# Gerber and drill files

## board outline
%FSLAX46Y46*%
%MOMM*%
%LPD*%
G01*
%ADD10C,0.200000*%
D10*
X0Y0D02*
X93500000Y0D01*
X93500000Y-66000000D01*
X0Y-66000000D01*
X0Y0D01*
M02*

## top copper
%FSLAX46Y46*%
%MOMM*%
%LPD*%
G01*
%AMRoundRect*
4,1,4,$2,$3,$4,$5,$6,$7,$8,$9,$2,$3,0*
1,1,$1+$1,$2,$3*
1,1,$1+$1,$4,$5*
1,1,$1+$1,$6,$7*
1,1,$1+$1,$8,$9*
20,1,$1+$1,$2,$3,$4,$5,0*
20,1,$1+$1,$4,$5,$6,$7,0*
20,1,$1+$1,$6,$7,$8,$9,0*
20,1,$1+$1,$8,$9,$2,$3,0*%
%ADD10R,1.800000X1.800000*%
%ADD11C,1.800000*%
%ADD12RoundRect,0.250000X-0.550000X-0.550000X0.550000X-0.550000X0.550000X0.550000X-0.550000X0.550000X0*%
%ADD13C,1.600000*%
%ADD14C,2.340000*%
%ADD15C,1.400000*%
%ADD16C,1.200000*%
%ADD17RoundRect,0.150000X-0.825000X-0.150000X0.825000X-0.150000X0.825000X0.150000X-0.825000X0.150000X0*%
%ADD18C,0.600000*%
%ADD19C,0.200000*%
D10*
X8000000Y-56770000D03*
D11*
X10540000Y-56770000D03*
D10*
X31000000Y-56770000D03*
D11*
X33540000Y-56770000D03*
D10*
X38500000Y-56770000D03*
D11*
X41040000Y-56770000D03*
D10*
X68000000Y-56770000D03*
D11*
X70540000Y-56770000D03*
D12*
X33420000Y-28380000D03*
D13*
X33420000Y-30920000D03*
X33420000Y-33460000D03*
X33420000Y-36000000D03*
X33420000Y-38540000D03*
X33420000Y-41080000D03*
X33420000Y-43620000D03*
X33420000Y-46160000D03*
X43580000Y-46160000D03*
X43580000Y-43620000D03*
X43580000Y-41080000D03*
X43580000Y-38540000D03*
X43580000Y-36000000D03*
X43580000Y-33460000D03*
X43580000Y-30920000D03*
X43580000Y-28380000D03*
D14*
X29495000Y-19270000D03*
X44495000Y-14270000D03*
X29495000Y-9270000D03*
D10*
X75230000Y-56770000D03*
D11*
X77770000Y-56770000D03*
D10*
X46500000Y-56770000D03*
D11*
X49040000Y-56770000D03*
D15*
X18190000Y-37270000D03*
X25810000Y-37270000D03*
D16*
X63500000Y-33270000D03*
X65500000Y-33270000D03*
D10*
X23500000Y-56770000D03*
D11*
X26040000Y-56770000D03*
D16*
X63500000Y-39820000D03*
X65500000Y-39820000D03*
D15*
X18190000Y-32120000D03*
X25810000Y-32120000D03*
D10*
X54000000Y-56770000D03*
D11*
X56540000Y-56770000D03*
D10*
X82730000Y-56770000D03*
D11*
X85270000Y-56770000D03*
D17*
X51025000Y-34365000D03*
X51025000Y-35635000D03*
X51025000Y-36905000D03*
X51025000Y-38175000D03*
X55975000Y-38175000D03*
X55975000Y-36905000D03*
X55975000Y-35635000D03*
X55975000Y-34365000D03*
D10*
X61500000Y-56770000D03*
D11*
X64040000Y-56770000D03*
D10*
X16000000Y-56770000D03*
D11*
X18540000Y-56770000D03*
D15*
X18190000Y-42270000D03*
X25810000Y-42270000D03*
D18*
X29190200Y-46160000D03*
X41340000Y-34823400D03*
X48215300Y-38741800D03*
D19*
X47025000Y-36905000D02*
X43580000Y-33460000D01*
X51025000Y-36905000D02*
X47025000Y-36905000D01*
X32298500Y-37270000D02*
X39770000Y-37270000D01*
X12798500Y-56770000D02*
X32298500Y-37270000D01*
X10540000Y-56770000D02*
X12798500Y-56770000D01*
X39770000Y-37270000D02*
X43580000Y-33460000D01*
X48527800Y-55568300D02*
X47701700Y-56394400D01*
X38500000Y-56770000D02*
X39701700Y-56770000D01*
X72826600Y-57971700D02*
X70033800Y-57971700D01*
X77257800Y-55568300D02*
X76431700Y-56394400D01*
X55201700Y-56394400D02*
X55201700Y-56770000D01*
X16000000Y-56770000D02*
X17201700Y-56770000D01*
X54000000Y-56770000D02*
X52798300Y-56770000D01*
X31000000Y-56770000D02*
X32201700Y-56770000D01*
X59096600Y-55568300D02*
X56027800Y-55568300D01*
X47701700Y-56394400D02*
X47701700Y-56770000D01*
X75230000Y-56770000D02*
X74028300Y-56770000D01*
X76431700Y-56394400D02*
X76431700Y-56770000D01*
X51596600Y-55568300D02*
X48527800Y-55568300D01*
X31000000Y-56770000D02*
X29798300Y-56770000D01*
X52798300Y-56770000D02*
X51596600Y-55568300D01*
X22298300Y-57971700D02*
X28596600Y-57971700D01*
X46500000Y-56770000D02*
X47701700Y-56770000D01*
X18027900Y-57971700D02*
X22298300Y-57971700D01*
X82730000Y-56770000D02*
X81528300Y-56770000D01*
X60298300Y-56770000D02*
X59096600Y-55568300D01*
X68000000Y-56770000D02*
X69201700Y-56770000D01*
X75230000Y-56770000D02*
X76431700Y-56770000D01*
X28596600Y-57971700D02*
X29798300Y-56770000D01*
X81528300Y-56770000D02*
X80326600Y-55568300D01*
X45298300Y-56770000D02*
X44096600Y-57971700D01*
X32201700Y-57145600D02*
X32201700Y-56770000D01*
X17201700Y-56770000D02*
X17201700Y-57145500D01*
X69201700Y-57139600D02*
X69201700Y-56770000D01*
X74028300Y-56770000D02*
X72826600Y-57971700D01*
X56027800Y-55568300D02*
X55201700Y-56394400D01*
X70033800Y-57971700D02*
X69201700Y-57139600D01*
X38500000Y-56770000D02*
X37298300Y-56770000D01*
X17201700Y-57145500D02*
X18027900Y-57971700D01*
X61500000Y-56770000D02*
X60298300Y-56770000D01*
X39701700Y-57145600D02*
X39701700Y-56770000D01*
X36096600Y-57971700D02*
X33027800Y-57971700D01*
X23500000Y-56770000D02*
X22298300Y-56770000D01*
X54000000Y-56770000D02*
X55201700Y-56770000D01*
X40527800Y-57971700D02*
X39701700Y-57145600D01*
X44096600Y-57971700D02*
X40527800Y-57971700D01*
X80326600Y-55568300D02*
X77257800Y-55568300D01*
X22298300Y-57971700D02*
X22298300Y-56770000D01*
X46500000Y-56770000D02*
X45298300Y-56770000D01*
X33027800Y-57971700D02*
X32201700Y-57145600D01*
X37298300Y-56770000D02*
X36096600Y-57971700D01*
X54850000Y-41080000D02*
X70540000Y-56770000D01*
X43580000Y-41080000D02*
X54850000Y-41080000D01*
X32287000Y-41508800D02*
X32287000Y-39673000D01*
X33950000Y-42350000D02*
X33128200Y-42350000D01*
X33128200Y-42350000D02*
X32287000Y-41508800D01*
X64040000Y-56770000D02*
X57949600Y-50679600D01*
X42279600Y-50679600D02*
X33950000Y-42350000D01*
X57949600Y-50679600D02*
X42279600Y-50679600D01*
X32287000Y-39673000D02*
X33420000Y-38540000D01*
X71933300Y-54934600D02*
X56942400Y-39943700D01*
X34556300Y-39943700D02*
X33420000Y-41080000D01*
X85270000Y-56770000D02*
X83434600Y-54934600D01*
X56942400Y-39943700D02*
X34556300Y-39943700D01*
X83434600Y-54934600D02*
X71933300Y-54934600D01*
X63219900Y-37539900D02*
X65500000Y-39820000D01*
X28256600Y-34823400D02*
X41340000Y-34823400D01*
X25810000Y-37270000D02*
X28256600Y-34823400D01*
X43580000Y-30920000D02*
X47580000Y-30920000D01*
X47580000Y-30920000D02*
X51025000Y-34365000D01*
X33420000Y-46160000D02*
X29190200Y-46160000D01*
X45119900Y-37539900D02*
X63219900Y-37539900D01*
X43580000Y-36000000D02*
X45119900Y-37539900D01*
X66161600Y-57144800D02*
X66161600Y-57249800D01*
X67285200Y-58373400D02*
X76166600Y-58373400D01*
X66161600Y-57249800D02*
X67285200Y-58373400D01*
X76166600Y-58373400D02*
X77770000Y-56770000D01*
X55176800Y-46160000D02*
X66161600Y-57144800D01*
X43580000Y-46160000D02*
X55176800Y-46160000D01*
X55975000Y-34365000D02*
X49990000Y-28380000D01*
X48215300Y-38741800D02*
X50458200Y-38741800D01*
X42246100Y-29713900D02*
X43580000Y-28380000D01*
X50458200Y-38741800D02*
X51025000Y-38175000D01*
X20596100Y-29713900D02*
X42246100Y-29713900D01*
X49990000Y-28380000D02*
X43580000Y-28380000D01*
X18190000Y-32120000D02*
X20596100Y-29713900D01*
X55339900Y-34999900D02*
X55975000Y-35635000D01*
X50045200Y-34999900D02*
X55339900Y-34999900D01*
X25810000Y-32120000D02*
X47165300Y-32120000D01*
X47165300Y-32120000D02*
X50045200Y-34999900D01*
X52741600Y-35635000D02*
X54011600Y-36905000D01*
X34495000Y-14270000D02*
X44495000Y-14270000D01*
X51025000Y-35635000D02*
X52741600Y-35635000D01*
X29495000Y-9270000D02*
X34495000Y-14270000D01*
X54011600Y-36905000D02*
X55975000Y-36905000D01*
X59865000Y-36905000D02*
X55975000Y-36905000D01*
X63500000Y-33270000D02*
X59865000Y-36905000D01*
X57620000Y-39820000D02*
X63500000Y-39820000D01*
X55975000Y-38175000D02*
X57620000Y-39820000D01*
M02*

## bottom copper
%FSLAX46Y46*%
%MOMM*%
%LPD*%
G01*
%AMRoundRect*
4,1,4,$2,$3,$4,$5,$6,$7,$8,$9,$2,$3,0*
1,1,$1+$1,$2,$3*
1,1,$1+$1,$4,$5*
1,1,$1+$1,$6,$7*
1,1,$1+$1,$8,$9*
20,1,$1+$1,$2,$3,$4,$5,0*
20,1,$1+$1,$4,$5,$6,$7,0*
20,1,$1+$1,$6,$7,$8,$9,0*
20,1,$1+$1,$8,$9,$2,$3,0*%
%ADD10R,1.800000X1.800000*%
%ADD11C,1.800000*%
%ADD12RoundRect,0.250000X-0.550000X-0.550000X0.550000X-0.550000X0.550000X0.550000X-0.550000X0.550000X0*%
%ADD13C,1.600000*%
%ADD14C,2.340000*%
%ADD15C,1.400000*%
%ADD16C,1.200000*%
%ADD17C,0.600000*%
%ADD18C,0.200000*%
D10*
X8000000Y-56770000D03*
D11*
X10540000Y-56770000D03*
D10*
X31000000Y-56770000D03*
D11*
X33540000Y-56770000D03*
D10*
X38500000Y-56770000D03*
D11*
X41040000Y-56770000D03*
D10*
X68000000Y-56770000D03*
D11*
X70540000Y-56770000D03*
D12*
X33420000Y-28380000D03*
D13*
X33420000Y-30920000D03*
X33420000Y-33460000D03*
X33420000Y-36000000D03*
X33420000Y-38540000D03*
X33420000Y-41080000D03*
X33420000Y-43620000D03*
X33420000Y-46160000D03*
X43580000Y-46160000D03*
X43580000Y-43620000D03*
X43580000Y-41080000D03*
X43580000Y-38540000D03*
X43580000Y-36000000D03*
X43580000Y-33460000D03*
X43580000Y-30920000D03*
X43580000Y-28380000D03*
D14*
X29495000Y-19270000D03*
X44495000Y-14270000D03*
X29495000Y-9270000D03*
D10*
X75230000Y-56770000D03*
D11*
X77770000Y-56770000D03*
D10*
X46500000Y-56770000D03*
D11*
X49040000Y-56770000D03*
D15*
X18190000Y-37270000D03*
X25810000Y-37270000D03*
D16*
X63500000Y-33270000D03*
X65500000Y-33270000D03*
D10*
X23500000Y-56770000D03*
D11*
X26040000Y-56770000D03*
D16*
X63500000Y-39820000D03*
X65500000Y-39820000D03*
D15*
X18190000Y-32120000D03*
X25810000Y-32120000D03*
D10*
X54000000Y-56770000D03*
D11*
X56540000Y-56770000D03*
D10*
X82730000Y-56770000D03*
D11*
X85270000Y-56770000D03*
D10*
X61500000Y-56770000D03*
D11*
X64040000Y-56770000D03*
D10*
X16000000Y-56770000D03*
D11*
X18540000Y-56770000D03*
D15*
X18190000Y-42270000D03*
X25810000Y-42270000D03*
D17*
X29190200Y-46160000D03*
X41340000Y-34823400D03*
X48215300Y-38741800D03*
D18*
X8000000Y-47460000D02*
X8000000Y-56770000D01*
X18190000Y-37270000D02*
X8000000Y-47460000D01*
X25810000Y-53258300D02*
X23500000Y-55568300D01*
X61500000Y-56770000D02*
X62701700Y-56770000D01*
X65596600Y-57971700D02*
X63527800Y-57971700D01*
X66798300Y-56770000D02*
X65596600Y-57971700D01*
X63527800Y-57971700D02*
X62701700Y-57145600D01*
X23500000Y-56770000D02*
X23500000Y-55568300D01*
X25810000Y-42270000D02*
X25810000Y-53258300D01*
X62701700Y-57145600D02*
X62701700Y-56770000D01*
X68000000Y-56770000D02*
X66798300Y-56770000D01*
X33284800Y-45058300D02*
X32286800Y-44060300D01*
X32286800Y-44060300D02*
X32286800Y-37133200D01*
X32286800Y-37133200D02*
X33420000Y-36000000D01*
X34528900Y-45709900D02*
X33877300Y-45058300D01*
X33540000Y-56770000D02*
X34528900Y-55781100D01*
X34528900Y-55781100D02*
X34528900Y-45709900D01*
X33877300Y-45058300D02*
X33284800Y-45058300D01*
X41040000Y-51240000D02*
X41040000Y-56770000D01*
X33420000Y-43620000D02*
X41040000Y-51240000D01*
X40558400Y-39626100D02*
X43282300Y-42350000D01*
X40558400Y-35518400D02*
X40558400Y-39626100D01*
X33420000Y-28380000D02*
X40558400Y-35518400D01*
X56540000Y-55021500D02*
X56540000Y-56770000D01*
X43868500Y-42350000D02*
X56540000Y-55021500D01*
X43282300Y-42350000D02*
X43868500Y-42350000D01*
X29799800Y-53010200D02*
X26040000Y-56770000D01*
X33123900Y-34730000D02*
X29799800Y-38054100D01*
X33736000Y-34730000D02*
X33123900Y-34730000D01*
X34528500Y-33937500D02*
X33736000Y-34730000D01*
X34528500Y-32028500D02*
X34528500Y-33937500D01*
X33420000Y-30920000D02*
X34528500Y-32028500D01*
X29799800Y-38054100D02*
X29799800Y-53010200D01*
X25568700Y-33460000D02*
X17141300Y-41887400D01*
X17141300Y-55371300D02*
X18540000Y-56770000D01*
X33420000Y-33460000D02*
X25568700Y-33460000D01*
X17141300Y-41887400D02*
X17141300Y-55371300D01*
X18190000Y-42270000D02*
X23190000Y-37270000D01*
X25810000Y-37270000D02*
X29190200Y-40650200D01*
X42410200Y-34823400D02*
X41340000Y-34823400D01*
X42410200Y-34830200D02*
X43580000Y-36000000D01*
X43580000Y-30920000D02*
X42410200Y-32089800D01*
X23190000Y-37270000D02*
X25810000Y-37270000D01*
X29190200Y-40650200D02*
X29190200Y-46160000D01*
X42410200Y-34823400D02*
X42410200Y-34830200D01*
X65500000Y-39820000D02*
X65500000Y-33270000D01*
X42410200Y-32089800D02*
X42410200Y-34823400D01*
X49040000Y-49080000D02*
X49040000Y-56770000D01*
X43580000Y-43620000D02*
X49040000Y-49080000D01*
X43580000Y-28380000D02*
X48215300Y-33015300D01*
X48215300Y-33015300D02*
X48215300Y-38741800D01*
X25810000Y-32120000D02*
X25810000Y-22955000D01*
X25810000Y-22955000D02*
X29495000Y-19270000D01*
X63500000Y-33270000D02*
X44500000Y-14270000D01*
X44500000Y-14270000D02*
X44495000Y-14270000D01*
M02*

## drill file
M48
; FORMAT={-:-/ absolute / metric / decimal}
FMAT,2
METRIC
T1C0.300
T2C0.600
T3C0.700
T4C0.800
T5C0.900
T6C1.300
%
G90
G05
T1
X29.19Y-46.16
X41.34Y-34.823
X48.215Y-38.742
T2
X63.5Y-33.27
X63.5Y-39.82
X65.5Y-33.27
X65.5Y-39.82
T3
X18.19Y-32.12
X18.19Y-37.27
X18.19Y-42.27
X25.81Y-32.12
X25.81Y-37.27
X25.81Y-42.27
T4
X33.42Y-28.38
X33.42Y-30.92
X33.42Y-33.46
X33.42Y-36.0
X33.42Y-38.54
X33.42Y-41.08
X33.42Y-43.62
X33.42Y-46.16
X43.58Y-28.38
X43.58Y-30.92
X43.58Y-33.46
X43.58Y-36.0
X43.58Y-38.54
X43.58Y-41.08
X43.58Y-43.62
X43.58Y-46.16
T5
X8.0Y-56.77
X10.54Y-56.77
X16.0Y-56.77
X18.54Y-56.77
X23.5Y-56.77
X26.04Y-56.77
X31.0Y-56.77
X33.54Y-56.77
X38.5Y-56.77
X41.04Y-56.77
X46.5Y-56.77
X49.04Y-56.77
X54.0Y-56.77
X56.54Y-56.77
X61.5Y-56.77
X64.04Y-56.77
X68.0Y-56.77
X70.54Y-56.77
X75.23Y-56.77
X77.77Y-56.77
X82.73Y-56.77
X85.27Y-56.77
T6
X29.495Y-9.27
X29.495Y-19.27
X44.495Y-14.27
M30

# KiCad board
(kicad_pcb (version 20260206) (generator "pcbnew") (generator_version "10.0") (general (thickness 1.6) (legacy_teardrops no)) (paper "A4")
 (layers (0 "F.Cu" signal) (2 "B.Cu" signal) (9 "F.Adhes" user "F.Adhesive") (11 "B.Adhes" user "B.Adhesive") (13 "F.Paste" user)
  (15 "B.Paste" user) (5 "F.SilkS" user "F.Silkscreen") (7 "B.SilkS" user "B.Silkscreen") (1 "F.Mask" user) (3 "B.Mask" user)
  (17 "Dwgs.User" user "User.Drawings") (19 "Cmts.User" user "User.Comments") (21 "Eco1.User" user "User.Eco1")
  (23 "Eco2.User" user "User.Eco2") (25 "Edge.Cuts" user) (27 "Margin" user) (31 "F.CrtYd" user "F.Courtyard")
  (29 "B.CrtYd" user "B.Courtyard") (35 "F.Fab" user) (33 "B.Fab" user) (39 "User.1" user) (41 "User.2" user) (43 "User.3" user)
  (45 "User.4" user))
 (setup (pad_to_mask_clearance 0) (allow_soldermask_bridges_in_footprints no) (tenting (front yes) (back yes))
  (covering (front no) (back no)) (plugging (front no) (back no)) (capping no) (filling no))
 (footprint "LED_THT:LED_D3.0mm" (layer "F.Cu") (at 8 56.77)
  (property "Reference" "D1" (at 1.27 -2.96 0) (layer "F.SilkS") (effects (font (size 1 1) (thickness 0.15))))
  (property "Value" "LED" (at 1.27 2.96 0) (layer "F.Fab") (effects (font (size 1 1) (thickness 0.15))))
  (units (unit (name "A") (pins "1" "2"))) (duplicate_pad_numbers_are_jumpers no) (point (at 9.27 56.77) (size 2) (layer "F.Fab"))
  (pad "1" thru_hole rect (at 0 0) (size 1.8 1.8) (drill 0.9) (layers "*.Cu" "*.Mask") (remove_unused_layers no) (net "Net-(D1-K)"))
  (pad "2" thru_hole circle (at 2.54 0) (size 1.8 1.8) (drill 0.9) (layers "*.Cu" "*.Mask") (remove_unused_layers no) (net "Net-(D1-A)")))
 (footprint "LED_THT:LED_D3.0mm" (layer "F.Cu") (at 31 56.77)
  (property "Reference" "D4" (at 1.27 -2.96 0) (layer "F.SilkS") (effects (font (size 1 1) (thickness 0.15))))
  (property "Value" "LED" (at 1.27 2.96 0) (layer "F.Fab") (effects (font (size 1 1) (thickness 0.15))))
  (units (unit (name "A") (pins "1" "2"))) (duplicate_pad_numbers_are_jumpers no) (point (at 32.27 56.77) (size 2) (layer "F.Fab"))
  (pad "1" thru_hole rect (at 0 0) (size 1.8 1.8) (drill 0.9) (layers "*.Cu" "*.Mask") (remove_unused_layers no) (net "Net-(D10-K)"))
  (pad "2" thru_hole circle (at 2.54 0) (size 1.8 1.8) (drill 0.9) (layers "*.Cu" "*.Mask") (remove_unused_layers no) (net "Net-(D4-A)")))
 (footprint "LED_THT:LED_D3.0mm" (layer "F.Cu") (at 38.5 56.77)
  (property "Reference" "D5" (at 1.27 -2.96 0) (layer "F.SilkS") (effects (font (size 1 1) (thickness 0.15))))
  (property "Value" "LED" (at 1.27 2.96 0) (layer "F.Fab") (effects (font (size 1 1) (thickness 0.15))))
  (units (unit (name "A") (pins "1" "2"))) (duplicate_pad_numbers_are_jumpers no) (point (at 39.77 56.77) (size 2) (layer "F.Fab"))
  (pad "1" thru_hole rect (at 0 0) (size 1.8 1.8) (drill 0.9) (layers "*.Cu" "*.Mask") (remove_unused_layers no) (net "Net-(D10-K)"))
  (pad "2" thru_hole circle (at 2.54 0) (size 1.8 1.8) (drill 0.9) (layers "*.Cu" "*.Mask") (remove_unused_layers no) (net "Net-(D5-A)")))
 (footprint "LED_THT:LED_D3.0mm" (layer "F.Cu") (at 68 56.77)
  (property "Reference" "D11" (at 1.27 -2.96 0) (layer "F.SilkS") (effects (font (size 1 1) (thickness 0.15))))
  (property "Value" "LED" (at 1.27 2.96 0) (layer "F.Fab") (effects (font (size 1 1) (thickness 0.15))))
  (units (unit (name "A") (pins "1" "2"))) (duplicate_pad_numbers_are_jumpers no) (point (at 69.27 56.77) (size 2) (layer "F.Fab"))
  (pad "1" thru_hole rect (at 0 0) (size 1.8 1.8) (drill 0.9) (layers "*.Cu" "*.Mask") (remove_unused_layers no) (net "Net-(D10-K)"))
  (pad "2" thru_hole circle (at 2.54 0) (size 1.8 1.8) (drill 0.9) (layers "*.Cu" "*.Mask") (remove_unused_layers no) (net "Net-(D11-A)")))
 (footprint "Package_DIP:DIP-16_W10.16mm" (layer "F.Cu") (at 33.42 28.38)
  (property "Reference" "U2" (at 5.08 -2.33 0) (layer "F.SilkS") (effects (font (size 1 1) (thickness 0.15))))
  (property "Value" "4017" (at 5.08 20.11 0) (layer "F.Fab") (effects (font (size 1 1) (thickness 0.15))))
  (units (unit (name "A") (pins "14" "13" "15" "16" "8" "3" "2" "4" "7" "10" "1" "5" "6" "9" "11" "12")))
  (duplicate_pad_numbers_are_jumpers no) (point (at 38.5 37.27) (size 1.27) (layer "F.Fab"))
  (pad "1" thru_hole roundrect (at 0 0) (size 1.6 1.6) (drill 0.8) (layers "*.Cu" "*.Mask") (remove_unused_layers no)
   (roundrect_rratio 0.15625) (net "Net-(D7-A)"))
  (pad "2" thru_hole circle (at 0 2.54) (size 1.6 1.6) (drill 0.8) (layers "*.Cu" "*.Mask") (remove_unused_layers no) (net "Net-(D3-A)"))
  (pad "3" thru_hole circle (at 0 5.08) (size 1.6 1.6) (drill 0.8) (layers "*.Cu" "*.Mask") (remove_unused_layers no) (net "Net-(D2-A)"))
  (pad "4" thru_hole circle (at 0 7.62) (size 1.6 1.6) (drill 0.8) (layers "*.Cu" "*.Mask") (remove_unused_layers no) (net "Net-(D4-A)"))
  (pad "5" thru_hole circle (at 0 10.16) (size 1.6 1.6) (drill 0.8) (layers "*.Cu" "*.Mask") (remove_unused_layers no) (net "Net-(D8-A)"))
  (pad "6" thru_hole circle (at 0 12.7) (size 1.6 1.6) (drill 0.8) (layers "*.Cu" "*.Mask") (remove_unused_layers no) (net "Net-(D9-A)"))
  (pad "7" thru_hole circle (at 0 15.24) (size 1.6 1.6) (drill 0.8) (layers "*.Cu" "*.Mask") (remove_unused_layers no) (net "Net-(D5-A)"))
  (pad "8" thru_hole circle (at 0 17.78) (size 1.6 1.6) (drill 0.8) (layers "*.Cu" "*.Mask") (remove_unused_layers no) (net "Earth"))
  (pad "9" thru_hole circle (at 10.16 17.78) (size 1.6 1.6) (drill 0.8) (layers "*.Cu" "*.Mask") (remove_unused_layers no)
   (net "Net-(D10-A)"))
  (pad "10" thru_hole circle (at 10.16 15.24) (size 1.6 1.6) (drill 0.8) (layers "*.Cu" "*.Mask") (remove_unused_layers no)
   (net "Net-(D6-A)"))
  (pad "11" thru_hole circle (at 10.16 12.7) (size 1.6 1.6) (drill 0.8) (layers "*.Cu" "*.Mask") (remove_unused_layers no)
   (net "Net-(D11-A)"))
  (pad "12" thru_hole circle (at 10.16 10.16) (size 1.6 1.6) (drill 0.8) (layers "*.Cu" "*.Mask") (remove_unused_layers no)
   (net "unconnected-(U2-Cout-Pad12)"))
  (pad "13" thru_hole circle (at 10.16 7.62) (size 1.6 1.6) (drill 0.8) (layers "*.Cu" "*.Mask") (remove_unused_layers no) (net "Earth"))
  (pad "14" thru_hole circle (at 10.16 5.08) (size 1.6 1.6) (drill 0.8) (layers "*.Cu" "*.Mask") (remove_unused_layers no)
   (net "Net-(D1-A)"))
  (pad "15" thru_hole circle (at 10.16 2.54) (size 1.6 1.6) (drill 0.8) (layers "*.Cu" "*.Mask") (remove_unused_layers no) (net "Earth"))
  (pad "16" thru_hole circle (at 10.16 0) (size 1.6 1.6) (drill 0.8) (layers "*.Cu" "*.Mask") (remove_unused_layers no) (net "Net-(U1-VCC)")))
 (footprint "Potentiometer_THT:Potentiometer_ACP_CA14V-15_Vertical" (layer "F.Cu") (at 29.495 19.27)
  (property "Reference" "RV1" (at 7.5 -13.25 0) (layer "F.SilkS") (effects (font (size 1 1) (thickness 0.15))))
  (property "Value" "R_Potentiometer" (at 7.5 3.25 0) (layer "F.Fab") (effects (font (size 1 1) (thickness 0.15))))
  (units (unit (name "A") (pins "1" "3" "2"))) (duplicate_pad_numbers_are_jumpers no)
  (pad "1" thru_hole circle (at 0 0) (size 2.34 2.34) (drill 1.3) (layers "*.Cu" "*.Mask") (remove_unused_layers no) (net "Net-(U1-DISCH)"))
  (pad "2" thru_hole circle (at 15 -5) (size 2.34 2.34) (drill 1.3) (layers "*.Cu" "*.Mask") (remove_unused_layers no)
   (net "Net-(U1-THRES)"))
  (pad "3" thru_hole circle (at 0 -10) (size 2.34 2.34) (drill 1.3) (layers "*.Cu" "*.Mask") (remove_unused_layers no)
   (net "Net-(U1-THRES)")))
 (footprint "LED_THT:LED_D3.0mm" (layer "F.Cu") (at 75.23 56.77)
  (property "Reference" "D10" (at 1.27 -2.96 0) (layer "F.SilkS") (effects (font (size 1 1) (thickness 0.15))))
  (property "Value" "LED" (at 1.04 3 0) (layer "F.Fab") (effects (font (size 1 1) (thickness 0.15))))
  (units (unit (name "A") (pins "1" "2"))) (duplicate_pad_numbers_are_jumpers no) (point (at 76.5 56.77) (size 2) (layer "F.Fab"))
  (pad "1" thru_hole rect (at 0 0) (size 1.8 1.8) (drill 0.9) (layers "*.Cu" "*.Mask") (remove_unused_layers no) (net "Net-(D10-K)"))
  (pad "2" thru_hole circle (at 2.54 0) (size 1.8 1.8) (drill 0.9) (layers "*.Cu" "*.Mask") (remove_unused_layers no) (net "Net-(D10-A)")))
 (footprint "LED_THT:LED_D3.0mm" (layer "F.Cu") (at 46.5 56.77)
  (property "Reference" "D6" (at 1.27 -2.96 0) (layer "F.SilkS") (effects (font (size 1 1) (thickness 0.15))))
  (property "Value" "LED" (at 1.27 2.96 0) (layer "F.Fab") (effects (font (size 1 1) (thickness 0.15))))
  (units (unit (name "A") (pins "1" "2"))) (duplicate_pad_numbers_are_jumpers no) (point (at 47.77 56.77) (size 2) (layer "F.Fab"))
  (pad "1" thru_hole rect (at 0 0) (size 1.8 1.8) (drill 0.9) (layers "*.Cu" "*.Mask") (remove_unused_layers no) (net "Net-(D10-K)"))
  (pad "2" thru_hole circle (at 2.54 0) (size 1.8 1.8) (drill 0.9) (layers "*.Cu" "*.Mask") (remove_unused_layers no) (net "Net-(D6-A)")))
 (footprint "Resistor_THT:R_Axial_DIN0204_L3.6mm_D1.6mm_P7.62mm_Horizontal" (layer "F.Cu") (at 18.19 37.27)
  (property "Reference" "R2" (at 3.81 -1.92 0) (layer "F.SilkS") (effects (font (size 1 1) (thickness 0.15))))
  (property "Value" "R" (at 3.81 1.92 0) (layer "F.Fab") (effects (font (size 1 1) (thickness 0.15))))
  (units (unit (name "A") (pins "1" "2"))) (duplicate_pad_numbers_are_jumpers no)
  (pad "1" thru_hole circle (at 0 0) (size 1.4 1.4) (drill 0.7) (layers "*.Cu" "*.Mask") (remove_unused_layers no) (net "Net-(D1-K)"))
  (pad "2" thru_hole circle (at 7.62 0) (size 1.4 1.4) (drill 0.7) (layers "*.Cu" "*.Mask") (remove_unused_layers no) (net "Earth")))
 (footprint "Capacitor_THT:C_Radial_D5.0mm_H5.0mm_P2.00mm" (layer "F.Cu") (at 63.5 33.27)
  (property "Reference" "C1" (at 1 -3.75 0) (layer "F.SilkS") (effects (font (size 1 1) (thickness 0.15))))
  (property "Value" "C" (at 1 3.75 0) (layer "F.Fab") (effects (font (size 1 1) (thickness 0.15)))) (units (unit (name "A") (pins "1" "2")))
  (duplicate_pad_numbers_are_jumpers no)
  (pad "1" thru_hole circle (at 0 0) (size 1.2 1.2) (drill 0.6) (layers "*.Cu" "*.Mask") (remove_unused_layers no) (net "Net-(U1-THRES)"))
  (pad "2" thru_hole circle (at 2 0) (size 1.2 1.2) (drill 0.6) (layers "*.Cu" "*.Mask") (remove_unused_layers no) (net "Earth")))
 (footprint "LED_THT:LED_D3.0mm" (layer "F.Cu") (at 23.5 56.77)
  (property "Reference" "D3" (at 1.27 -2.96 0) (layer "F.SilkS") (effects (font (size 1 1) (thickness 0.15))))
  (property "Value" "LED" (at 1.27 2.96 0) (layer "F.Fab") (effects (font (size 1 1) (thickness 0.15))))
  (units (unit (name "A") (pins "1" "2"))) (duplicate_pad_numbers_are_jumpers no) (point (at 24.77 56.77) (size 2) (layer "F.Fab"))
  (pad "1" thru_hole rect (at 0 0) (size 1.8 1.8) (drill 0.9) (layers "*.Cu" "*.Mask") (remove_unused_layers no) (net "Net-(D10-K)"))
  (pad "2" thru_hole circle (at 2.54 0) (size 1.8 1.8) (drill 0.9) (layers "*.Cu" "*.Mask") (remove_unused_layers no) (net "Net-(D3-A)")))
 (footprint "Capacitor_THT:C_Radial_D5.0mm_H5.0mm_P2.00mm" (layer "F.Cu") (at 63.5 39.82)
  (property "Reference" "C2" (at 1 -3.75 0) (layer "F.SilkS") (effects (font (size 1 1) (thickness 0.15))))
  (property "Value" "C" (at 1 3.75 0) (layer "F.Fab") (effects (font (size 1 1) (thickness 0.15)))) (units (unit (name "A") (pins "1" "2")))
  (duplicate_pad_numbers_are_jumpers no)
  (pad "1" thru_hole circle (at 0 0) (size 1.2 1.2) (drill 0.6) (layers "*.Cu" "*.Mask") (remove_unused_layers no) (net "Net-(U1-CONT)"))
  (pad "2" thru_hole circle (at 2 0) (size 1.2 1.2) (drill 0.6) (layers "*.Cu" "*.Mask") (remove_unused_layers no) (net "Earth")))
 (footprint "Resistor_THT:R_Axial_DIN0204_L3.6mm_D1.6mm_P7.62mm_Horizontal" (layer "F.Cu") (at 18.19 32.12)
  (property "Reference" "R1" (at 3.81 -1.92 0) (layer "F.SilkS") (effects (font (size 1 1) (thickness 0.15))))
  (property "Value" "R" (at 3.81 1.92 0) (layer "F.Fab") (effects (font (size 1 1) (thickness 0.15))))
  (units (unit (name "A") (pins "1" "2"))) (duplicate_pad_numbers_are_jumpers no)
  (pad "1" thru_hole circle (at 0 0) (size 1.4 1.4) (drill 0.7) (layers "*.Cu" "*.Mask") (remove_unused_layers no) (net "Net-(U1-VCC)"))
  (pad "2" thru_hole circle (at 7.62 0) (size 1.4 1.4) (drill 0.7) (layers "*.Cu" "*.Mask") (remove_unused_layers no) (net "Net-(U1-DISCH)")))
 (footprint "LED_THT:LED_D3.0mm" (layer "F.Cu") (at 54 56.77)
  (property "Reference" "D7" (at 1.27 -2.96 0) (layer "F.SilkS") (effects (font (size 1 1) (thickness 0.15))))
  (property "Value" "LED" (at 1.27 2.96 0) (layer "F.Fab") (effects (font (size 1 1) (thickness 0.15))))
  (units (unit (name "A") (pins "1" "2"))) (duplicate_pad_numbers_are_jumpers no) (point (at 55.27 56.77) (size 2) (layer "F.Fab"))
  (pad "1" thru_hole rect (at 0 0) (size 1.8 1.8) (drill 0.9) (layers "*.Cu" "*.Mask") (remove_unused_layers no) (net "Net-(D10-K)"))
  (pad "2" thru_hole circle (at 2.54 0) (size 1.8 1.8) (drill 0.9) (layers "*.Cu" "*.Mask") (remove_unused_layers no) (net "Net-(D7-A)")))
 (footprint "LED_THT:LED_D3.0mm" (layer "F.Cu") (at 82.73 56.77)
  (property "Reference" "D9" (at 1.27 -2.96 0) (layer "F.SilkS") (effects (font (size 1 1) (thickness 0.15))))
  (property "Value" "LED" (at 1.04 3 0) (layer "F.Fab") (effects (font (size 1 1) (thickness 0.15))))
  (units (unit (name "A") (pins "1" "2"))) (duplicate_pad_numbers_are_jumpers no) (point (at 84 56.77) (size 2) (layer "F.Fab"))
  (pad "1" thru_hole rect (at 0 0) (size 1.8 1.8) (drill 0.9) (layers "*.Cu" "*.Mask") (remove_unused_layers no) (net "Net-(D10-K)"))
  (pad "2" thru_hole circle (at 2.54 0) (size 1.8 1.8) (drill 0.9) (layers "*.Cu" "*.Mask") (remove_unused_layers no) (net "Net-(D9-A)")))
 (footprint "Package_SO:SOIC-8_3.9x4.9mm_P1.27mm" (layer "F.Cu") (at 53.5 36.27)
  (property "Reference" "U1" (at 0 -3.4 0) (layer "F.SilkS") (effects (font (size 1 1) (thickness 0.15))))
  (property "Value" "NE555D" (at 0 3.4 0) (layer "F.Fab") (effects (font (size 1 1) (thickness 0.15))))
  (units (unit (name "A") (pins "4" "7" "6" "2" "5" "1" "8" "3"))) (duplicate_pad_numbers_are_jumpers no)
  (pad "1" smd roundrect (at -2.475 -1.905) (size 1.95 0.6) (layers "F.Cu" "F.Mask" "F.Paste") (roundrect_rratio 0.25) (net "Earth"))
  (pad "2" smd roundrect (at -2.475 -0.635) (size 1.95 0.6) (layers "F.Cu" "F.Mask" "F.Paste") (roundrect_rratio 0.25)
   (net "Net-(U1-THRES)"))
  (pad "3" smd roundrect (at -2.475 0.635) (size 1.95 0.6) (layers "F.Cu" "F.Mask" "F.Paste") (roundrect_rratio 0.25) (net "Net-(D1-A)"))
  (pad "4" smd roundrect (at -2.475 1.905) (size 1.95 0.6) (layers "F.Cu" "F.Mask" "F.Paste") (roundrect_rratio 0.25) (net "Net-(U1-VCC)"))
  (pad "5" smd roundrect (at 2.475 1.905) (size 1.95 0.6) (layers "F.Cu" "F.Mask" "F.Paste") (roundrect_rratio 0.25) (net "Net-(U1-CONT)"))
  (pad "6" smd roundrect (at 2.475 0.635) (size 1.95 0.6) (layers "F.Cu" "F.Mask" "F.Paste") (roundrect_rratio 0.25) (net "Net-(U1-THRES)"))
  (pad "7" smd roundrect (at 2.475 -0.635) (size 1.95 0.6) (layers "F.Cu" "F.Mask" "F.Paste") (roundrect_rratio 0.25) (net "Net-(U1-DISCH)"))
  (pad "8" smd roundrect (at 2.475 -1.905) (size 1.95 0.6) (layers "F.Cu" "F.Mask" "F.Paste") (roundrect_rratio 0.25) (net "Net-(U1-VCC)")))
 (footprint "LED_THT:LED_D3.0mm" (layer "F.Cu") (at 61.5 56.77)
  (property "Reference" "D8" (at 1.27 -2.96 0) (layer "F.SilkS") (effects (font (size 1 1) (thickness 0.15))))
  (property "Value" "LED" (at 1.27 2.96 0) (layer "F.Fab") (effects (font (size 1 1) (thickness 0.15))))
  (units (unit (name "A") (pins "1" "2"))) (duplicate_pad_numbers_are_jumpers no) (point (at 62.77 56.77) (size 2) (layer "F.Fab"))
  (pad "1" thru_hole rect (at 0 0) (size 1.8 1.8) (drill 0.9) (layers "*.Cu" "*.Mask") (remove_unused_layers no) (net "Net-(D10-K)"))
  (pad "2" thru_hole circle (at 2.54 0) (size 1.8 1.8) (drill 0.9) (layers "*.Cu" "*.Mask") (remove_unused_layers no) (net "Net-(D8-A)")))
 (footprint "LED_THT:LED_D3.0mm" (layer "F.Cu") (at 16 56.77)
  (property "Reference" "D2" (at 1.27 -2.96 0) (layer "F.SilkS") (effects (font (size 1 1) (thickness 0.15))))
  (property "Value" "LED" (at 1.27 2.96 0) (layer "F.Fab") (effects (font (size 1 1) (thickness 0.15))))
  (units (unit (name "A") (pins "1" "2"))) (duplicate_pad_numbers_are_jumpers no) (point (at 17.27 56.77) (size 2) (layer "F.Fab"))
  (pad "1" thru_hole rect (at 0 0) (size 1.8 1.8) (drill 0.9) (layers "*.Cu" "*.Mask") (remove_unused_layers no) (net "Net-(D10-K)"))
  (pad "2" thru_hole circle (at 2.54 0) (size 1.8 1.8) (drill 0.9) (layers "*.Cu" "*.Mask") (remove_unused_layers no) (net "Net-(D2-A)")))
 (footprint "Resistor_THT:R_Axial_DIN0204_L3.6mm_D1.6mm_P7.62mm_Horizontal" (layer "F.Cu") (at 18.19 42.27)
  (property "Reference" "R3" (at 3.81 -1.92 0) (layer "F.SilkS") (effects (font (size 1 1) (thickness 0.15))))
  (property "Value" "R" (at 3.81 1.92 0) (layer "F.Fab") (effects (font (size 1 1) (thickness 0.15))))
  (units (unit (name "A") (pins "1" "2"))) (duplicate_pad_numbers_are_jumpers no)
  (pad "1" thru_hole circle (at 0 0) (size 1.4 1.4) (drill 0.7) (layers "*.Cu" "*.Mask") (remove_unused_layers no) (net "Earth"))
  (pad "2" thru_hole circle (at 7.62 0) (size 1.4 1.4) (drill 0.7) (layers "*.Cu" "*.Mask") (remove_unused_layers no) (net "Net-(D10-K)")))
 (gr_rect (start 0 0) (end 93.5 66) (stroke (width 0.2) (type solid)) (fill no) (layer "Edge.Cuts"))
 (segment (start 8 47.46) (end 8 56.77) (width 0.2) (layer "B.Cu") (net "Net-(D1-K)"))
 (segment (start 18.19 37.27) (end 8 47.46) (width 0.2) (layer "B.Cu") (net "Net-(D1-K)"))
 (segment (start 47.025 36.905) (end 43.58 33.46) (width 0.2) (layer "F.Cu") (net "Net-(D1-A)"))
 (segment (start 51.025 36.905) (end 47.025 36.905) (width 0.2) (layer "F.Cu") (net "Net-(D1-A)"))
 (segment (start 32.2985 37.27) (end 39.77 37.27) (width 0.2) (layer "F.Cu") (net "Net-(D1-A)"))
 (segment (start 12.7985 56.77) (end 32.2985 37.27) (width 0.2) (layer "F.Cu") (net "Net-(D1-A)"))
 (segment (start 10.54 56.77) (end 12.7985 56.77) (width 0.2) (layer "F.Cu") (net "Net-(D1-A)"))
 (segment (start 39.77 37.27) (end 43.58 33.46) (width 0.2) (layer "F.Cu") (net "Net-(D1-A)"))
 (segment (start 48.5278 55.5683) (end 47.7017 56.3944) (width 0.2) (layer "F.Cu") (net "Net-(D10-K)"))
 (segment (start 38.5 56.77) (end 39.7017 56.77) (width 0.2) (layer "F.Cu") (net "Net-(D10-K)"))
 (segment (start 72.8266 57.9717) (end 70.0338 57.9717) (width 0.2) (layer "F.Cu") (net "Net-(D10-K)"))
 (segment (start 77.2578 55.5683) (end 76.4317 56.3944) (width 0.2) (layer "F.Cu") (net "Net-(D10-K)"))
 (segment (start 55.2017 56.3944) (end 55.2017 56.77) (width 0.2) (layer "F.Cu") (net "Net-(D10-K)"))
 (segment (start 16 56.77) (end 17.2017 56.77) (width 0.2) (layer "F.Cu") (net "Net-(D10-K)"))
 (segment (start 54 56.77) (end 52.7983 56.77) (width 0.2) (layer "F.Cu") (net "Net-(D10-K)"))
 (segment (start 31 56.77) (end 32.2017 56.77) (width 0.2) (layer "F.Cu") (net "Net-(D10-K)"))
 (segment (start 59.0966 55.5683) (end 56.0278 55.5683) (width 0.2) (layer "F.Cu") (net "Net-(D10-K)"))
 (segment (start 47.7017 56.3944) (end 47.7017 56.77) (width 0.2) (layer "F.Cu") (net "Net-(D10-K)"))
 (segment (start 75.23 56.77) (end 74.0283 56.77) (width 0.2) (layer "F.Cu") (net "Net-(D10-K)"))
 (segment (start 76.4317 56.3944) (end 76.4317 56.77) (width 0.2) (layer "F.Cu") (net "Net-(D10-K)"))
 (segment (start 51.5966 55.5683) (end 48.5278 55.5683) (width 0.2) (layer "F.Cu") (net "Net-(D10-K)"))
 (segment (start 31 56.77) (end 29.7983 56.77) (width 0.2) (layer "F.Cu") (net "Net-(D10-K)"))
 (segment (start 52.7983 56.77) (end 51.5966 55.5683) (width 0.2) (layer "F.Cu") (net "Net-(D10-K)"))
 (segment (start 22.2983 57.9717) (end 28.5966 57.9717) (width 0.2) (layer "F.Cu") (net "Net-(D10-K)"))
 (segment (start 46.5 56.77) (end 47.7017 56.77) (width 0.2) (layer "F.Cu") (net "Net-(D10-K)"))
 (segment (start 18.0279 57.9717) (end 22.2983 57.9717) (width 0.2) (layer "F.Cu") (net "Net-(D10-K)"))
 (segment (start 82.73 56.77) (end 81.5283 56.77) (width 0.2) (layer "F.Cu") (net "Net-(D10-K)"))
 (segment (start 60.2983 56.77) (end 59.0966 55.5683) (width 0.2) (layer "F.Cu") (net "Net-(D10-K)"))
 (segment (start 68 56.77) (end 69.2017 56.77) (width 0.2) (layer "F.Cu") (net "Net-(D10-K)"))
 (segment (start 75.23 56.77) (end 76.4317 56.77) (width 0.2) (layer "F.Cu") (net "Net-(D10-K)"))
 (segment (start 28.5966 57.9717) (end 29.7983 56.77) (width 0.2) (layer "F.Cu") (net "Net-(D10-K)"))
 (segment (start 81.5283 56.77) (end 80.3266 55.5683) (width 0.2) (layer "F.Cu") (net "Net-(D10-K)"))
 (segment (start 45.2983 56.77) (end 44.0966 57.9717) (width 0.2) (layer "F.Cu") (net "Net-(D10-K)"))
 (segment (start 32.2017 57.1456) (end 32.2017 56.77) (width 0.2) (layer "F.Cu") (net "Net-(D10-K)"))
 (segment (start 17.2017 56.77) (end 17.2017 57.1455) (width 0.2) (layer "F.Cu") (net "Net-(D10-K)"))
 (segment (start 69.2017 57.1396) (end 69.2017 56.77) (width 0.2) (layer "F.Cu") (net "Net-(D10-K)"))
 (segment (start 74.0283 56.77) (end 72.8266 57.9717) (width 0.2) (layer "F.Cu") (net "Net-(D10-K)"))
 (segment (start 56.0278 55.5683) (end 55.2017 56.3944) (width 0.2) (layer "F.Cu") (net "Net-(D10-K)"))
 (segment (start 70.0338 57.9717) (end 69.2017 57.1396) (width 0.2) (layer "F.Cu") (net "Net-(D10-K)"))
 (segment (start 38.5 56.77) (end 37.2983 56.77) (width 0.2) (layer "F.Cu") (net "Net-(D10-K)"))
 (segment (start 17.2017 57.1455) (end 18.0279 57.9717) (width 0.2) (layer "F.Cu") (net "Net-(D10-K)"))
 (segment (start 61.5 56.77) (end 60.2983 56.77) (width 0.2) (layer "F.Cu") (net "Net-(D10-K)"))
 (segment (start 39.7017 57.1456) (end 39.7017 56.77) (width 0.2) (layer "F.Cu") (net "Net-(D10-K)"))
 (segment (start 36.0966 57.9717) (end 33.0278 57.9717) (width 0.2) (layer "F.Cu") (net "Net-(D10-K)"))
 (segment (start 23.5 56.77) (end 22.2983 56.77) (width 0.2) (layer "F.Cu") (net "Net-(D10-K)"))
 (segment (start 54 56.77) (end 55.2017 56.77) (width 0.2) (layer "F.Cu") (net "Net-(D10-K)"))
 (segment (start 40.5278 57.9717) (end 39.7017 57.1456) (width 0.2) (layer "F.Cu") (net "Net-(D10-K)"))
 (segment (start 44.0966 57.9717) (end 40.5278 57.9717) (width 0.2) (layer "F.Cu") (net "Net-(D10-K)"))
 (segment (start 80.3266 55.5683) (end 77.2578 55.5683) (width 0.2) (layer "F.Cu") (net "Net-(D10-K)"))
 (segment (start 22.2983 57.9717) (end 22.2983 56.77) (width 0.2) (layer "F.Cu") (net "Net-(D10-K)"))
 (segment (start 46.5 56.77) (end 45.2983 56.77) (width 0.2) (layer "F.Cu") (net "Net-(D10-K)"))
 (segment (start 33.0278 57.9717) (end 32.2017 57.1456) (width 0.2) (layer "F.Cu") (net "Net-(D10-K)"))
 (segment (start 37.2983 56.77) (end 36.0966 57.9717) (width 0.2) (layer "F.Cu") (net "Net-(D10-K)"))
 (segment (start 25.81 53.2583) (end 23.5 55.5683) (width 0.2) (layer "B.Cu") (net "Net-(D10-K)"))
 (segment (start 61.5 56.77) (end 62.7017 56.77) (width 0.2) (layer "B.Cu") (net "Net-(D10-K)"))
 (segment (start 65.5966 57.9717) (end 63.5278 57.9717) (width 0.2) (layer "B.Cu") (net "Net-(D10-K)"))
 (segment (start 66.7983 56.77) (end 65.5966 57.9717) (width 0.2) (layer "B.Cu") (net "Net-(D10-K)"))
 (segment (start 63.5278 57.9717) (end 62.7017 57.1456) (width 0.2) (layer "B.Cu") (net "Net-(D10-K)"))
 (segment (start 23.5 56.77) (end 23.5 55.5683) (width 0.2) (layer "B.Cu") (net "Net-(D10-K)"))
 (segment (start 25.81 42.27) (end 25.81 53.2583) (width 0.2) (layer "B.Cu") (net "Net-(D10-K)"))
 (segment (start 62.7017 57.1456) (end 62.7017 56.77) (width 0.2) (layer "B.Cu") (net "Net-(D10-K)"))
 (segment (start 68 56.77) (end 66.7983 56.77) (width 0.2) (layer "B.Cu") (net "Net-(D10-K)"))
 (segment (start 33.2848 45.0583) (end 32.2868 44.0603) (width 0.2) (layer "B.Cu") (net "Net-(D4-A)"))
 (segment (start 32.2868 44.0603) (end 32.2868 37.1332) (width 0.2) (layer "B.Cu") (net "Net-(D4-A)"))
 (segment (start 32.2868 37.1332) (end 33.42 36) (width 0.2) (layer "B.Cu") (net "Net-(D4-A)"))
 (segment (start 34.5289 45.7099) (end 33.8773 45.0583) (width 0.2) (layer "B.Cu") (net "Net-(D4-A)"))
 (segment (start 33.54 56.77) (end 34.5289 55.7811) (width 0.2) (layer "B.Cu") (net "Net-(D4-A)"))
 (segment (start 34.5289 55.7811) (end 34.5289 45.7099) (width 0.2) (layer "B.Cu") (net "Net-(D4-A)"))
 (segment (start 33.8773 45.0583) (end 33.2848 45.0583) (width 0.2) (layer "B.Cu") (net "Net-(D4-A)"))
 (segment (start 41.04 51.24) (end 41.04 56.77) (width 0.2) (layer "B.Cu") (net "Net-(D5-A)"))
 (segment (start 33.42 43.62) (end 41.04 51.24) (width 0.2) (layer "B.Cu") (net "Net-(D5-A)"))
 (segment (start 54.85 41.08) (end 70.54 56.77) (width 0.2) (layer "F.Cu") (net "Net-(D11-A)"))
 (segment (start 43.58 41.08) (end 54.85 41.08) (width 0.2) (layer "F.Cu") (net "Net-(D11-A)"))
 (segment (start 40.5584 39.6261) (end 43.2823 42.35) (width 0.2) (layer "B.Cu") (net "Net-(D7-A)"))
 (segment (start 40.5584 35.5184) (end 40.5584 39.6261) (width 0.2) (layer "B.Cu") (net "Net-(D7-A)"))
 (segment (start 33.42 28.38) (end 40.5584 35.5184) (width 0.2) (layer "B.Cu") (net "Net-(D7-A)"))
 (segment (start 56.54 55.0215) (end 56.54 56.77) (width 0.2) (layer "B.Cu") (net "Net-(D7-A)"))
 (segment (start 43.8685 42.35) (end 56.54 55.0215) (width 0.2) (layer "B.Cu") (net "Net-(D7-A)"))
 (segment (start 43.2823 42.35) (end 43.8685 42.35) (width 0.2) (layer "B.Cu") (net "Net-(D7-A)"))
 (segment (start 29.7998 53.0102) (end 26.04 56.77) (width 0.2) (layer "B.Cu") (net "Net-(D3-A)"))
 (segment (start 33.1239 34.73) (end 29.7998 38.0541) (width 0.2) (layer "B.Cu") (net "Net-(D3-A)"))
 (segment (start 33.736 34.73) (end 33.1239 34.73) (width 0.2) (layer "B.Cu") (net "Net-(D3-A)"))
 (segment (start 34.5285 33.9375) (end 33.736 34.73) (width 0.2) (layer "B.Cu") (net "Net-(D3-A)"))
 (segment (start 34.5285 32.0285) (end 34.5285 33.9375) (width 0.2) (layer "B.Cu") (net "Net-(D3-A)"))
 (segment (start 33.42 30.92) (end 34.5285 32.0285) (width 0.2) (layer "B.Cu") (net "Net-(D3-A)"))
 (segment (start 29.7998 38.0541) (end 29.7998 53.0102) (width 0.2) (layer "B.Cu") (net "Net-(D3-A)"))
 (segment (start 25.5687 33.46) (end 17.1413 41.8874) (width 0.2) (layer "B.Cu") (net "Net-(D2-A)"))
 (segment (start 17.1413 55.3713) (end 18.54 56.77) (width 0.2) (layer "B.Cu") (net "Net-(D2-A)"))
 (segment (start 33.42 33.46) (end 25.5687 33.46) (width 0.2) (layer "B.Cu") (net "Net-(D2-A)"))
 (segment (start 17.1413 41.8874) (end 17.1413 55.3713) (width 0.2) (layer "B.Cu") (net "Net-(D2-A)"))
 (segment (start 32.287 41.5088) (end 32.287 39.673) (width 0.2) (layer "F.Cu") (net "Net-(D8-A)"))
 (segment (start 33.95 42.35) (end 33.1282 42.35) (width 0.2) (layer "F.Cu") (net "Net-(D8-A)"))
 (segment (start 33.1282 42.35) (end 32.287 41.5088) (width 0.2) (layer "F.Cu") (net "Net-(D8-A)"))
 (segment (start 64.04 56.77) (end 57.9496 50.6796) (width 0.2) (layer "F.Cu") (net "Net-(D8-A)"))
 (segment (start 42.2796 50.6796) (end 33.95 42.35) (width 0.2) (layer "F.Cu") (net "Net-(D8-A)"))
 (segment (start 57.9496 50.6796) (end 42.2796 50.6796) (width 0.2) (layer "F.Cu") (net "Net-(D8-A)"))
 (segment (start 32.287 39.673) (end 33.42 38.54) (width 0.2) (layer "F.Cu") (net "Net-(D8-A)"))
 (segment (start 71.9333 54.9346) (end 56.9424 39.9437) (width 0.2) (layer "F.Cu") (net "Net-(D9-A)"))
 (segment (start 34.5563 39.9437) (end 33.42 41.08) (width 0.2) (layer "F.Cu") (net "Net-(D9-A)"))
 (segment (start 85.27 56.77) (end 83.4346 54.9346) (width 0.2) (layer "F.Cu") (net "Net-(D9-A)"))
 (segment (start 56.9424 39.9437) (end 34.5563 39.9437) (width 0.2) (layer "F.Cu") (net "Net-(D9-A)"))
 (segment (start 83.4346 54.9346) (end 71.9333 54.9346) (width 0.2) (layer "F.Cu") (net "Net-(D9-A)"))
 (segment (start 63.2199 37.5399) (end 65.5 39.82) (width 0.2) (layer "F.Cu") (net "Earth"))
 (segment (start 28.2566 34.8234) (end 41.34 34.8234) (width 0.2) (layer "F.Cu") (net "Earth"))
 (segment (start 25.81 37.27) (end 28.2566 34.8234) (width 0.2) (layer "F.Cu") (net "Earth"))
 (segment (start 43.58 30.92) (end 47.58 30.92) (width 0.2) (layer "F.Cu") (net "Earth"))
 (segment (start 47.58 30.92) (end 51.025 34.365) (width 0.2) (layer "F.Cu") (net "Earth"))
 (segment (start 33.42 46.16) (end 29.1902 46.16) (width 0.2) (layer "F.Cu") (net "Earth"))
 (segment (start 45.1199 37.5399) (end 63.2199 37.5399) (width 0.2) (layer "F.Cu") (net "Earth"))
 (segment (start 43.58 36) (end 45.1199 37.5399) (width 0.2) (layer "F.Cu") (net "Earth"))
 (via (at 29.1902 46.16) (size 0.6) (drill 0.3) (layers "F.Cu" "B.Cu") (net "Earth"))
 (via (at 41.34 34.8234) (size 0.6) (drill 0.3) (layers "F.Cu" "B.Cu") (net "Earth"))
 (segment (start 18.19 42.27) (end 23.19 37.27) (width 0.2) (layer "B.Cu") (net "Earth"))
 (segment (start 25.81 37.27) (end 29.1902 40.6502) (width 0.2) (layer "B.Cu") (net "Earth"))
 (segment (start 42.4102 34.8234) (end 41.34 34.8234) (width 0.2) (layer "B.Cu") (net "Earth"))
 (segment (start 42.4102 34.8302) (end 43.58 36) (width 0.2) (layer "B.Cu") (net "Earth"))
 (segment (start 43.58 30.92) (end 42.4102 32.0898) (width 0.2) (layer "B.Cu") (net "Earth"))
 (segment (start 23.19 37.27) (end 25.81 37.27) (width 0.2) (layer "B.Cu") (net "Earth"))
 (segment (start 29.1902 40.6502) (end 29.1902 46.16) (width 0.2) (layer "B.Cu") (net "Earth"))
 (segment (start 42.4102 34.8234) (end 42.4102 34.8302) (width 0.2) (layer "B.Cu") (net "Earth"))
 (segment (start 65.5 39.82) (end 65.5 33.27) (width 0.2) (layer "B.Cu") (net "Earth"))
 (segment (start 42.4102 32.0898) (end 42.4102 34.8234) (width 0.2) (layer "B.Cu") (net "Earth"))
 (segment (start 66.1616 57.1448) (end 66.1616 57.2498) (width 0.2) (layer "F.Cu") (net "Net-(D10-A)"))
 (segment (start 67.2852 58.3734) (end 76.1666 58.3734) (width 0.2) (layer "F.Cu") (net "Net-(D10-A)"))
 (segment (start 66.1616 57.2498) (end 67.2852 58.3734) (width 0.2) (layer "F.Cu") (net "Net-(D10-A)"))
 (segment (start 76.1666 58.3734) (end 77.77 56.77) (width 0.2) (layer "F.Cu") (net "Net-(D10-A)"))
 (segment (start 55.1768 46.16) (end 66.1616 57.1448) (width 0.2) (layer "F.Cu") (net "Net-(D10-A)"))
 (segment (start 43.58 46.16) (end 55.1768 46.16) (width 0.2) (layer "F.Cu") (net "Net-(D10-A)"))
 (segment (start 49.04 49.08) (end 49.04 56.77) (width 0.2) (layer "B.Cu") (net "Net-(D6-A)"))
 (segment (start 43.58 43.62) (end 49.04 49.08) (width 0.2) (layer "B.Cu") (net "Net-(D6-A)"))
 (segment (start 55.975 34.365) (end 49.99 28.38) (width 0.2) (layer "F.Cu") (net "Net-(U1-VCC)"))
 (segment (start 48.2153 38.7418) (end 50.4582 38.7418) (width 0.2) (layer "F.Cu") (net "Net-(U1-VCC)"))
 (segment (start 42.2461 29.7139) (end 43.58 28.38) (width 0.2) (layer "F.Cu") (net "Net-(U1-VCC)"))
 (segment (start 50.4582 38.7418) (end 51.025 38.175) (width 0.2) (layer "F.Cu") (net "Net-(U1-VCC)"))
 (segment (start 20.5961 29.7139) (end 42.2461 29.7139) (width 0.2) (layer "F.Cu") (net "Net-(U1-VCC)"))
 (segment (start 49.99 28.38) (end 43.58 28.38) (width 0.2) (layer "F.Cu") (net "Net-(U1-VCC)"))
 (segment (start 18.19 32.12) (end 20.5961 29.7139) (width 0.2) (layer "F.Cu") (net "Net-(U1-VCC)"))
 (via (at 48.2153 38.7418) (size 0.6) (drill 0.3) (layers "F.Cu" "B.Cu") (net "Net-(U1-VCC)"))
 (segment (start 43.58 28.38) (end 48.2153 33.0153) (width 0.2) (layer "B.Cu") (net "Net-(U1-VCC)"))
 (segment (start 48.2153 33.0153) (end 48.2153 38.7418) (width 0.2) (layer "B.Cu") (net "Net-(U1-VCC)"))
 (segment (start 55.3399 34.9999) (end 55.975 35.635) (width 0.2) (layer "F.Cu") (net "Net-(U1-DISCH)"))
 (segment (start 50.0452 34.9999) (end 55.3399 34.9999) (width 0.2) (layer "F.Cu") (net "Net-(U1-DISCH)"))
 (segment (start 25.81 32.12) (end 47.1653 32.12) (width 0.2) (layer "F.Cu") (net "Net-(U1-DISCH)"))
 (segment (start 47.1653 32.12) (end 50.0452 34.9999) (width 0.2) (layer "F.Cu") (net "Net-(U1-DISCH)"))
 (segment (start 25.81 32.12) (end 25.81 22.955) (width 0.2) (layer "B.Cu") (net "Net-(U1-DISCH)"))
 (segment (start 25.81 22.955) (end 29.495 19.27) (width 0.2) (layer "B.Cu") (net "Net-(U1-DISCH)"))
 (segment (start 52.7416 35.635) (end 54.0116 36.905) (width 0.2) (layer "F.Cu") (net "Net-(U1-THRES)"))
 (segment (start 34.495 14.27) (end 44.495 14.27) (width 0.2) (layer "F.Cu") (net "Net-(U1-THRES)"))
 (segment (start 51.025 35.635) (end 52.7416 35.635) (width 0.2) (layer "F.Cu") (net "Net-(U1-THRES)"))
 (segment (start 29.495 9.27) (end 34.495 14.27) (width 0.2) (layer "F.Cu") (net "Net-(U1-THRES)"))
 (segment (start 54.0116 36.905) (end 55.975 36.905) (width 0.2) (layer "F.Cu") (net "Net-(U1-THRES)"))
 (segment (start 59.865 36.905) (end 55.975 36.905) (width 0.2) (layer "F.Cu") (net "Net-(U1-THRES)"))
 (segment (start 63.5 33.27) (end 59.865 36.905) (width 0.2) (layer "F.Cu") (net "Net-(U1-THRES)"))
 (segment (start 63.5 33.27) (end 44.5 14.27) (width 0.2) (layer "B.Cu") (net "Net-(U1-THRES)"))
 (segment (start 44.5 14.27) (end 44.495 14.27) (width 0.2) (layer "B.Cu") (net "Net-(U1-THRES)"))
 (segment (start 57.62 39.82) (end 63.5 39.82) (width 0.2) (layer "F.Cu") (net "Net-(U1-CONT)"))
 (segment (start 55.975 38.175) (end 57.62 39.82) (width 0.2) (layer "F.Cu") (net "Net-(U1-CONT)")))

